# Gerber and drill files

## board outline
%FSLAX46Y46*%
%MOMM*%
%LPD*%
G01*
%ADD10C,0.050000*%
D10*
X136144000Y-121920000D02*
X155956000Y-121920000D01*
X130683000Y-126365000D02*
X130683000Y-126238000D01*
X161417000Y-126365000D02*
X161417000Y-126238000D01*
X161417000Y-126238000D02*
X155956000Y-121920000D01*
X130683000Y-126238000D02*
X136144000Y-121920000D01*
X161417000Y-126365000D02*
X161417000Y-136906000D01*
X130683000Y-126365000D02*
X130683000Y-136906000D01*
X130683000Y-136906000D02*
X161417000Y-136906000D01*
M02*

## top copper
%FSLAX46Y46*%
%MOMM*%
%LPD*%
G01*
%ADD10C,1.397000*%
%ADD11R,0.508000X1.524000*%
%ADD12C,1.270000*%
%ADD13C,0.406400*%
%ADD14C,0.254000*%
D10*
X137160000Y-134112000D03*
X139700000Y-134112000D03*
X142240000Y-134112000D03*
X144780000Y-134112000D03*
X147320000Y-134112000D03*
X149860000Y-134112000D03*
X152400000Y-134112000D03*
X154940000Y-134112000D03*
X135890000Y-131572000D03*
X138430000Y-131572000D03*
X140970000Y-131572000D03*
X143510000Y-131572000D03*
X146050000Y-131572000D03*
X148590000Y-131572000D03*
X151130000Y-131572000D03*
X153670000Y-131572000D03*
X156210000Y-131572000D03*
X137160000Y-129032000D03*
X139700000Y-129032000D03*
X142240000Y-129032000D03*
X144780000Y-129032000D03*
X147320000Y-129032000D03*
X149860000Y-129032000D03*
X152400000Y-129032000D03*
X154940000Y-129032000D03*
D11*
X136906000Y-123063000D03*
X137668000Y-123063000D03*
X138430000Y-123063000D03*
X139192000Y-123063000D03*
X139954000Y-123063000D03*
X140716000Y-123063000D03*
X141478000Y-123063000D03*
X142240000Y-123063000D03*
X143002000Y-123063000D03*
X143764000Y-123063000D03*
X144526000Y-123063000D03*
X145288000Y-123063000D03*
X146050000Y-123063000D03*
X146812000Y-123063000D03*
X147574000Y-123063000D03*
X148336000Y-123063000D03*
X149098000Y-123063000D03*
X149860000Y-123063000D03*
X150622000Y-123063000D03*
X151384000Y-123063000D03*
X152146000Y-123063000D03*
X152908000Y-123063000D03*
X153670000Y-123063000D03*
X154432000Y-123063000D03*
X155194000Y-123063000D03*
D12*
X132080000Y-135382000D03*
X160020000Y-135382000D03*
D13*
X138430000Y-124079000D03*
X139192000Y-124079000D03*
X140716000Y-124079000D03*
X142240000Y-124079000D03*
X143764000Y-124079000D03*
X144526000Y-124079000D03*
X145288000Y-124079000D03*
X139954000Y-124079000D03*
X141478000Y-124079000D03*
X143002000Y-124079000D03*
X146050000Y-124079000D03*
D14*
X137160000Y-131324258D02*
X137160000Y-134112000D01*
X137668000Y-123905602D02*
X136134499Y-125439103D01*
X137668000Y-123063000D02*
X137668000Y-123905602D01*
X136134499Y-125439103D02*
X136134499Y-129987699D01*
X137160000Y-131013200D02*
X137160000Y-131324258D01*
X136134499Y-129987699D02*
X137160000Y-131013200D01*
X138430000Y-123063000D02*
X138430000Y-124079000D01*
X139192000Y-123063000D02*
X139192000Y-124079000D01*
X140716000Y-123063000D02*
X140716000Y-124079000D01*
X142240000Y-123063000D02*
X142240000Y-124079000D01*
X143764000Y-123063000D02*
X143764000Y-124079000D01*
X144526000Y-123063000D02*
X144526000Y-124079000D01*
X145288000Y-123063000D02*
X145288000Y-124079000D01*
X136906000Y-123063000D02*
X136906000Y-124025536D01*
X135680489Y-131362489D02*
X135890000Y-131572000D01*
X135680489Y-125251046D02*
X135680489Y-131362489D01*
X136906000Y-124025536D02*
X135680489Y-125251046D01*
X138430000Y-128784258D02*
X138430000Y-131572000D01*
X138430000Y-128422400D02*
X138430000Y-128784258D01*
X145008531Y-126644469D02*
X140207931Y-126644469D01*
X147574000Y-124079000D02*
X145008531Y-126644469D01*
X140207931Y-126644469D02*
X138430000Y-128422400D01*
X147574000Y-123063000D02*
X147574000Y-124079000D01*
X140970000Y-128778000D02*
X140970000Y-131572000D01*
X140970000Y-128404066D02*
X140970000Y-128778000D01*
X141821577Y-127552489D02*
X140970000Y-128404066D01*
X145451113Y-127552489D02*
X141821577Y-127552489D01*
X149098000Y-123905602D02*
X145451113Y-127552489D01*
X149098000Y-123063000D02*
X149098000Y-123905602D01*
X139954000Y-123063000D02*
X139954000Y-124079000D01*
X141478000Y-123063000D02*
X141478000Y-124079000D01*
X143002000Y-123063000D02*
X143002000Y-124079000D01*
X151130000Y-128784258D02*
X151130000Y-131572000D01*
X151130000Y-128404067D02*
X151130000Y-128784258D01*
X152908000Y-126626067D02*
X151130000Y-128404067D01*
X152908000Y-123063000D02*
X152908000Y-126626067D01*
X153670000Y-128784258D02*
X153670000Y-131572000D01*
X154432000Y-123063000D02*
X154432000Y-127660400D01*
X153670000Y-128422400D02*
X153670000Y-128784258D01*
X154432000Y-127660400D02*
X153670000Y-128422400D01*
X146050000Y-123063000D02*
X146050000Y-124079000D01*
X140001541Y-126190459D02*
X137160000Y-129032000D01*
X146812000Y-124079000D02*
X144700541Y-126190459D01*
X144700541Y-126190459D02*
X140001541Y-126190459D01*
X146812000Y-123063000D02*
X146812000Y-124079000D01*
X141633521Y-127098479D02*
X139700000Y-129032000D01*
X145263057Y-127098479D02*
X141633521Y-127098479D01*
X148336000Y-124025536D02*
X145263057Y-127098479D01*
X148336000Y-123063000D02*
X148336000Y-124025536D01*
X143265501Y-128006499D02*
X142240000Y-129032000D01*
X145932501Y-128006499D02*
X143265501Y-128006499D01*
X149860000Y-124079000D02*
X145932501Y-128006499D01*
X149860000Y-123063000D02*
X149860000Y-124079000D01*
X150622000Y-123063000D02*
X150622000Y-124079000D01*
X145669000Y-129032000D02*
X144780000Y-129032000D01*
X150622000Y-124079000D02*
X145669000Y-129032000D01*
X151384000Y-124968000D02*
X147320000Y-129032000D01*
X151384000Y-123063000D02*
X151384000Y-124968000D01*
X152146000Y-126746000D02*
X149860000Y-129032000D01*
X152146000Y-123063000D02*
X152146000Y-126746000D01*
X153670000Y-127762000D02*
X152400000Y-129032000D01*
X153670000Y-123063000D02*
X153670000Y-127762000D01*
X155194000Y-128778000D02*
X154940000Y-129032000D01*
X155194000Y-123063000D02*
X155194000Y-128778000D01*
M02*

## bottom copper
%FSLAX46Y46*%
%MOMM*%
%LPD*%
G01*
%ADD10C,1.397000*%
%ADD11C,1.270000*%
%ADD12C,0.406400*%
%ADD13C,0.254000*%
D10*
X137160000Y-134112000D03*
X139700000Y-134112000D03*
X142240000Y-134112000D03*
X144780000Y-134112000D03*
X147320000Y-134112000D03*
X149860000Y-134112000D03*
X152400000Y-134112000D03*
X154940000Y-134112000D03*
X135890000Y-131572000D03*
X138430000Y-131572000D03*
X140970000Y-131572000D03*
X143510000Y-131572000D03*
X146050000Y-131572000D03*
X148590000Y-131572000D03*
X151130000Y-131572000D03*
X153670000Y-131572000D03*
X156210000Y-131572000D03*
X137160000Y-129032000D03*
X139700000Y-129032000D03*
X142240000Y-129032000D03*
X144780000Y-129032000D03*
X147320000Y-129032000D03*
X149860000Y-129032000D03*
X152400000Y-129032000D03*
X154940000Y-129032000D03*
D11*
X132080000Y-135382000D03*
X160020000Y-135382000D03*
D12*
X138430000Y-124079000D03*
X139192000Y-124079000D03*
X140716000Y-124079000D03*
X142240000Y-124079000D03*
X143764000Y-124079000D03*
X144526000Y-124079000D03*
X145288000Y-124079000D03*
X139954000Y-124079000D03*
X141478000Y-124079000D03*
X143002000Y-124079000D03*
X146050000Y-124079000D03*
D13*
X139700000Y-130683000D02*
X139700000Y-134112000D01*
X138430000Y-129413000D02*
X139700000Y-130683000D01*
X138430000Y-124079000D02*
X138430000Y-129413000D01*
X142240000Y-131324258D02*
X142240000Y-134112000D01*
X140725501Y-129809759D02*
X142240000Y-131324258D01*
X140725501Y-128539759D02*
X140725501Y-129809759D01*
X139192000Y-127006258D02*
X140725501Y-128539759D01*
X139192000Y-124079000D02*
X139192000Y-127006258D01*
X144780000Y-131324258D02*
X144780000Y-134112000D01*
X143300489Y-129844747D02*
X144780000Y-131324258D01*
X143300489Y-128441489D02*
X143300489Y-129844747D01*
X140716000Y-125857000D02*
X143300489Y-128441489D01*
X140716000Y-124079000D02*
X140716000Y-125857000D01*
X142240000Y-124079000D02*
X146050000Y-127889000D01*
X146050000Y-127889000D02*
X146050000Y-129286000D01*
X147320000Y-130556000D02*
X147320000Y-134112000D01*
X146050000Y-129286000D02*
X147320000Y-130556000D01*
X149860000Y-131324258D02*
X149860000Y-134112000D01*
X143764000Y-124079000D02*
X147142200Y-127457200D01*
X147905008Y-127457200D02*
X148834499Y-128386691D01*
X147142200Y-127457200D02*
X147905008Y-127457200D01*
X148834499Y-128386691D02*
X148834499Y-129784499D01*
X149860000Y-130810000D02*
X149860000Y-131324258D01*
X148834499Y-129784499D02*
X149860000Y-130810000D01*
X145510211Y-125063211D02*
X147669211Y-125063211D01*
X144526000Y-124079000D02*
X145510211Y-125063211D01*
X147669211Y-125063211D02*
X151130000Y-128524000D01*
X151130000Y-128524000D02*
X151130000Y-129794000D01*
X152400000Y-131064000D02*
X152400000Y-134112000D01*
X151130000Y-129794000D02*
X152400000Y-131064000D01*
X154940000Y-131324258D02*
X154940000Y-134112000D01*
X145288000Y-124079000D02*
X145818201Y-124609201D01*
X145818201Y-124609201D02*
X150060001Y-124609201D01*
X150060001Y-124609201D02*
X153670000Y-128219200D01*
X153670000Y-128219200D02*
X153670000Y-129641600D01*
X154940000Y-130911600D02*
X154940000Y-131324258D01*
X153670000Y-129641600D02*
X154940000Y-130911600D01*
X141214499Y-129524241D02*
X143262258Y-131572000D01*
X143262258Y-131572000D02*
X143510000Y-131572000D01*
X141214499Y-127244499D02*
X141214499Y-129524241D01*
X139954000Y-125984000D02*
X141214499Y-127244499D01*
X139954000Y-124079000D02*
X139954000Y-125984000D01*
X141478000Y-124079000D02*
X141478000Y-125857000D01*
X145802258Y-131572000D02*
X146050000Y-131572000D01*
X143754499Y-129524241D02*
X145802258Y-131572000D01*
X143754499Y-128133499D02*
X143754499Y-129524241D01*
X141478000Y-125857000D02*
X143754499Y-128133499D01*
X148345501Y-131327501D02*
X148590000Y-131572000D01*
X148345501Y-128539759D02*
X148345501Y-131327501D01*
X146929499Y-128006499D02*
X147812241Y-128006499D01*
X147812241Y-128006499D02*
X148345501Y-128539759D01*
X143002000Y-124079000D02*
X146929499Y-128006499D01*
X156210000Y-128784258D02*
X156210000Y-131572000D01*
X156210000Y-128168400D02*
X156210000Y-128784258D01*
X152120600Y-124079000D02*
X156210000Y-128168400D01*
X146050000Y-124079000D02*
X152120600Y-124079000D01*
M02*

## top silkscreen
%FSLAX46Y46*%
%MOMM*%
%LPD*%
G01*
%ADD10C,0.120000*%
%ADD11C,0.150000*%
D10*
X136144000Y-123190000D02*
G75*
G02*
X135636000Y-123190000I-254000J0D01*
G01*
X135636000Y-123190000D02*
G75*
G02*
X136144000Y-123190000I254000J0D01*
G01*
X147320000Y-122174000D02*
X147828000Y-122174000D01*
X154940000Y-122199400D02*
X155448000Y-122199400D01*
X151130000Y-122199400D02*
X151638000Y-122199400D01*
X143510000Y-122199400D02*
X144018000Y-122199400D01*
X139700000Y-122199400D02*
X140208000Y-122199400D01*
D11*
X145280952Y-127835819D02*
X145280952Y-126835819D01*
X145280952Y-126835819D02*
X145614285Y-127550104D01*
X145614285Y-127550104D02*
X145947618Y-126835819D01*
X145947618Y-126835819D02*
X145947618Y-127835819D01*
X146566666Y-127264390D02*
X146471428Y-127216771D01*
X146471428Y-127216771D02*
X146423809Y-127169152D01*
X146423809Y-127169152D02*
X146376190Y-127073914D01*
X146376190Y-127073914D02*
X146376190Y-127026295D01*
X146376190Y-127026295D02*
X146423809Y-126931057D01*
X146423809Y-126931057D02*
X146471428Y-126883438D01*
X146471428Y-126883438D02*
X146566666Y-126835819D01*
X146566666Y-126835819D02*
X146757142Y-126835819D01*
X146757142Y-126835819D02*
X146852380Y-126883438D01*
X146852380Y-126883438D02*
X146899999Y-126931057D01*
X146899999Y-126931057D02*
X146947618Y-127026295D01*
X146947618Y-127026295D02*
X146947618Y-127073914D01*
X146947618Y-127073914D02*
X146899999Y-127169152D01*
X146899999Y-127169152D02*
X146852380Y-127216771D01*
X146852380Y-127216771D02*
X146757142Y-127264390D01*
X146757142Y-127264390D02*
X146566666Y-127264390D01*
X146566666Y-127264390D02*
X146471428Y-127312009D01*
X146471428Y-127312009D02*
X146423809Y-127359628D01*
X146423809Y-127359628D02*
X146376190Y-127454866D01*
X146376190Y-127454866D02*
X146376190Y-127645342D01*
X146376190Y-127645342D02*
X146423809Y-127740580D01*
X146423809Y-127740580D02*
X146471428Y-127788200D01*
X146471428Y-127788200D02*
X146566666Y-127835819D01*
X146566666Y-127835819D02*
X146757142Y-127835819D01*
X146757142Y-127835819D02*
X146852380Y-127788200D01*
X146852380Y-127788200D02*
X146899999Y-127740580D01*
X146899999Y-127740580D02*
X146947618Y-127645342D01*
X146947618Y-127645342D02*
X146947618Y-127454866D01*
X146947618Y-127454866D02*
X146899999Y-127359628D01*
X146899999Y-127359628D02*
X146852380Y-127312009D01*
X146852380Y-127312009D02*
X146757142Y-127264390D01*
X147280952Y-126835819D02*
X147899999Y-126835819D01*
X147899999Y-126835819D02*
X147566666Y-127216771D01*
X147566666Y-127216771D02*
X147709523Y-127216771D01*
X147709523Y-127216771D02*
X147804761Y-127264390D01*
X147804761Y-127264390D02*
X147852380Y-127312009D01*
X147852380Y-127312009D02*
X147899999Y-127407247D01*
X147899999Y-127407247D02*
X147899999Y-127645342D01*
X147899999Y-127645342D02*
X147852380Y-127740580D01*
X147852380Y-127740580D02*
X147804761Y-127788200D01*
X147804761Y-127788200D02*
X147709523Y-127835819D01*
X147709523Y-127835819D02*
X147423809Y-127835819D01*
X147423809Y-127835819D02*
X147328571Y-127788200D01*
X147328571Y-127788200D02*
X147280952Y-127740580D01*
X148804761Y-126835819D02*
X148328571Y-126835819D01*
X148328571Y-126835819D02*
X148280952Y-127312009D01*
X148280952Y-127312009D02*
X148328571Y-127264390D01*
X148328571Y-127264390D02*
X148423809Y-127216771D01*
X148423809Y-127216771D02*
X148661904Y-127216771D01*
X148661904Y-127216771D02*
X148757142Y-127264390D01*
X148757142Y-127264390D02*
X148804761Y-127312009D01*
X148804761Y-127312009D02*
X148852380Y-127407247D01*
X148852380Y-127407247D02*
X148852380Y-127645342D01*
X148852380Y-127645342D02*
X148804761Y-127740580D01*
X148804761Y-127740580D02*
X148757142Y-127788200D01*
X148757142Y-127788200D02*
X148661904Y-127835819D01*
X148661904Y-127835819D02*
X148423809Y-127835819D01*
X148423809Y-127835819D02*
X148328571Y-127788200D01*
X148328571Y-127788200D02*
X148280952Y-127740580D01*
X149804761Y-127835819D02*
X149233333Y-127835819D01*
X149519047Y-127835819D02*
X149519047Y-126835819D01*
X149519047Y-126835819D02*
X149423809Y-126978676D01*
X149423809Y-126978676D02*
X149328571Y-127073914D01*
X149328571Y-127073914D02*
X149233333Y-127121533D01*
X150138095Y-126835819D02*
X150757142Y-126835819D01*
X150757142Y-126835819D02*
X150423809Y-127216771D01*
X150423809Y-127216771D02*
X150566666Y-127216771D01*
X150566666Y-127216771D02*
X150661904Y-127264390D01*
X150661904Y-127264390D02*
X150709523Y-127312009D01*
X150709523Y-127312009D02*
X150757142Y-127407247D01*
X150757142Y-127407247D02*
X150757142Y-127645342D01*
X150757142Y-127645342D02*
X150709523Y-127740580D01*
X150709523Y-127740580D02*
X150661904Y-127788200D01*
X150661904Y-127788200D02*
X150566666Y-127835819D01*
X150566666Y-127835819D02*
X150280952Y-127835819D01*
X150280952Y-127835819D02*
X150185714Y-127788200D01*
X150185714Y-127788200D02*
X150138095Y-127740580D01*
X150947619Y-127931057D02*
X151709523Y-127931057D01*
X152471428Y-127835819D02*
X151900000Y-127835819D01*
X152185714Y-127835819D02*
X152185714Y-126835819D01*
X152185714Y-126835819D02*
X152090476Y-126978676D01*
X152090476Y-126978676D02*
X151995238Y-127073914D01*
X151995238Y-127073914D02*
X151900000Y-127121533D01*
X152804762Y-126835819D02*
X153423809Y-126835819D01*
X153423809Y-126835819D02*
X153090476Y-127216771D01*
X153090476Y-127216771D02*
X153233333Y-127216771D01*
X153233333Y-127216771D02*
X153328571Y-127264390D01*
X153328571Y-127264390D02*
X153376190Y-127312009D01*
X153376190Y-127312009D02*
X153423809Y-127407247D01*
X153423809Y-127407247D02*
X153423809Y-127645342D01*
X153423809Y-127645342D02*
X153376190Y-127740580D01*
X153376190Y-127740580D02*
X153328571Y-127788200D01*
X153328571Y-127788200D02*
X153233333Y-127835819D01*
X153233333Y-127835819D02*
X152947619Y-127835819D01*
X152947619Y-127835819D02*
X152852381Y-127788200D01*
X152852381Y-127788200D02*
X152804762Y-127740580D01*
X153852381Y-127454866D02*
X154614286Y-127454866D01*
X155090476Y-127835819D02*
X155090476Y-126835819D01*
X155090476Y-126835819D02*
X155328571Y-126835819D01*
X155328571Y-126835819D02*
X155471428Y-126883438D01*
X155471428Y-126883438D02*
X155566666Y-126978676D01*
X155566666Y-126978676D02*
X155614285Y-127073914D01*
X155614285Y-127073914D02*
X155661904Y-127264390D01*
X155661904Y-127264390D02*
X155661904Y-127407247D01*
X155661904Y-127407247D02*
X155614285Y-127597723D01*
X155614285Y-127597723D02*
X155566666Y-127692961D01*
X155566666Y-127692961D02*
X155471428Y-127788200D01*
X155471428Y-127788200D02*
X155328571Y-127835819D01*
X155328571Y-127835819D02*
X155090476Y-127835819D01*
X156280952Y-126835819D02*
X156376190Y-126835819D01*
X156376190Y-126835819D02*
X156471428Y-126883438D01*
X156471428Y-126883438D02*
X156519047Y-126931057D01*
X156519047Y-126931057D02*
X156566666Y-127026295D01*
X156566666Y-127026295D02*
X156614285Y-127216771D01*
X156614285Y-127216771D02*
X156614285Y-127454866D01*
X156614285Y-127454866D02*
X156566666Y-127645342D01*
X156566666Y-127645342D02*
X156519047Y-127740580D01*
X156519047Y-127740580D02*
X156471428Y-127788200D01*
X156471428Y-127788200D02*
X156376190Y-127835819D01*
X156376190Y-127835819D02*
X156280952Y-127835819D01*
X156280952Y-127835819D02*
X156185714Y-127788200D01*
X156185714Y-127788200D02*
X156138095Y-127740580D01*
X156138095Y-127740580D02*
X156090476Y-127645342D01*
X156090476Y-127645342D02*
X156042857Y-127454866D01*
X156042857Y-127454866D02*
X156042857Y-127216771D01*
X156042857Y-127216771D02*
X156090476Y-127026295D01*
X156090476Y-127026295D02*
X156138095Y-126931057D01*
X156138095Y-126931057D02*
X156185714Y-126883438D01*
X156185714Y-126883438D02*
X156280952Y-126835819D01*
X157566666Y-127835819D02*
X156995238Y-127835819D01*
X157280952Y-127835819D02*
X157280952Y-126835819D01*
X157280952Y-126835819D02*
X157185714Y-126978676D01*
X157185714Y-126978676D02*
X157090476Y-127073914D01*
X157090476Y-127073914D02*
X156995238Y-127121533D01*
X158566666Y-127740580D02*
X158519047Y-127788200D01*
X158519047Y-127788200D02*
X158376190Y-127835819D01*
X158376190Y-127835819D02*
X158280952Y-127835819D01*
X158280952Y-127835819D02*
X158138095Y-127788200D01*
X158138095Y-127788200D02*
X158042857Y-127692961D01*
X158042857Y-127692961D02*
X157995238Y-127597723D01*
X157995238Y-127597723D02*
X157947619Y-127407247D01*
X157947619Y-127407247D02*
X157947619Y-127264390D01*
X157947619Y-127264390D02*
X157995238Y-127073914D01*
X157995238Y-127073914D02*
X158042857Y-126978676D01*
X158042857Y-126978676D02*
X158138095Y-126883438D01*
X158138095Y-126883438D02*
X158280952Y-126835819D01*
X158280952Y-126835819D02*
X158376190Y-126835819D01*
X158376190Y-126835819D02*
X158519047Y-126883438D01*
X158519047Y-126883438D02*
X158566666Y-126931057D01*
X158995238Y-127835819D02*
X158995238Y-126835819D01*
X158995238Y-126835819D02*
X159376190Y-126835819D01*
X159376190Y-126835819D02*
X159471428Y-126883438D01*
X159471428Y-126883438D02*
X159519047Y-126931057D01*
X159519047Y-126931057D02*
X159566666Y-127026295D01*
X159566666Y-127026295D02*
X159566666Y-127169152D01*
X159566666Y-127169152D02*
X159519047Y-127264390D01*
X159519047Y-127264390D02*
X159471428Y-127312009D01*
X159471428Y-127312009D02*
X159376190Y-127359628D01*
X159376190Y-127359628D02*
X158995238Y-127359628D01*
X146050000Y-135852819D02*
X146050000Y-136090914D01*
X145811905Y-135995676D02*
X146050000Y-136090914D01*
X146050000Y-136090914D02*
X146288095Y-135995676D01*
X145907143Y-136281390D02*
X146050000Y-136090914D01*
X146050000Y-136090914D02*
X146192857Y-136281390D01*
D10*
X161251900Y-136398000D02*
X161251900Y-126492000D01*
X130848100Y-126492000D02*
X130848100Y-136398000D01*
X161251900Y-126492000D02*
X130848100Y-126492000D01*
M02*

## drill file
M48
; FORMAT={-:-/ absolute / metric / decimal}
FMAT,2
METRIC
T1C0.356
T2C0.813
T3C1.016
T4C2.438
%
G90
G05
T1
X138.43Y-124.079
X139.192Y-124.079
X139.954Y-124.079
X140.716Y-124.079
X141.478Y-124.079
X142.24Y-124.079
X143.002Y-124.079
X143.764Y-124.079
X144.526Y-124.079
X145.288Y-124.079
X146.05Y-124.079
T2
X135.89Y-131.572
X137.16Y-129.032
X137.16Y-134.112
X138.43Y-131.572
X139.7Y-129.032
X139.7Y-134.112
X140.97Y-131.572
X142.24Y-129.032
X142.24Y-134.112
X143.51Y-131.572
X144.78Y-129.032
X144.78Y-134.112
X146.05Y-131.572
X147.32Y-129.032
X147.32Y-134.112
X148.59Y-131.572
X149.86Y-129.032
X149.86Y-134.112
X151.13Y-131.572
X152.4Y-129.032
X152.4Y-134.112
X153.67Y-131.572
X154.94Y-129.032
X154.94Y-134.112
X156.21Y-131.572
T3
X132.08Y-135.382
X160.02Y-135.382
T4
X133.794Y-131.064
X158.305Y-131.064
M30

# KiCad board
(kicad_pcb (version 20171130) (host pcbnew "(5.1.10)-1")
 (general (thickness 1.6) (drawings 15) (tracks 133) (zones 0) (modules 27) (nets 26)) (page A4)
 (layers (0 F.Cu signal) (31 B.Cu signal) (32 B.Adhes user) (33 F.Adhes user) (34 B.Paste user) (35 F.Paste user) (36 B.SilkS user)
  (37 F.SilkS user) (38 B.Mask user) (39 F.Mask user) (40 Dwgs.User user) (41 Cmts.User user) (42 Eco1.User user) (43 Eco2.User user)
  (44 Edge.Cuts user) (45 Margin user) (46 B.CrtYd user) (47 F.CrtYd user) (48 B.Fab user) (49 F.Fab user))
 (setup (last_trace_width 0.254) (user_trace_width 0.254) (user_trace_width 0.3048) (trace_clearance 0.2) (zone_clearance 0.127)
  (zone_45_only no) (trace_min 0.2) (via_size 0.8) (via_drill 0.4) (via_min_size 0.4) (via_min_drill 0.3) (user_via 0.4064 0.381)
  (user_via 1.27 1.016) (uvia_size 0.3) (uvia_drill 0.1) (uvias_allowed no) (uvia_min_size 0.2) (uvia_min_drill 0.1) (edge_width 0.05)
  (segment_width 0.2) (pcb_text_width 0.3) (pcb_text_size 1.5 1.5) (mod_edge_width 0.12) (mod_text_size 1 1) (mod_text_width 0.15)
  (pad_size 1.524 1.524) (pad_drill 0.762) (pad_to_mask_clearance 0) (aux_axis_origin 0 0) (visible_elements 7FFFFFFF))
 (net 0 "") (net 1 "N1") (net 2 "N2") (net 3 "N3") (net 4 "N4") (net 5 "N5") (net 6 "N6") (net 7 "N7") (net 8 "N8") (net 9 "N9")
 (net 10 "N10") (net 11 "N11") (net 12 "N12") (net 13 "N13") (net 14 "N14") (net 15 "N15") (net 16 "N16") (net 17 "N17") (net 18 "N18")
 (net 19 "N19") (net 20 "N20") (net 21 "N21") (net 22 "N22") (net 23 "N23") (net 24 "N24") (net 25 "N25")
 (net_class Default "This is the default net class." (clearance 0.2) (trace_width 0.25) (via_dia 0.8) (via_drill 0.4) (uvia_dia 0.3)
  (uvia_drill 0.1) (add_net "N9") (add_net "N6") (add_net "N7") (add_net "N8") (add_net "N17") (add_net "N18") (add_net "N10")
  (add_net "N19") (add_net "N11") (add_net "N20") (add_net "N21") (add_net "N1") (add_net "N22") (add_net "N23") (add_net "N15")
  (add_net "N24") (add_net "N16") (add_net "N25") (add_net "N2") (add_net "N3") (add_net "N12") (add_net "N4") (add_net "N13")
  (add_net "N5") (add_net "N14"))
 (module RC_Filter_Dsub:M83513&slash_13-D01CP (layer F.Cu) (at 146.05 137.414 180)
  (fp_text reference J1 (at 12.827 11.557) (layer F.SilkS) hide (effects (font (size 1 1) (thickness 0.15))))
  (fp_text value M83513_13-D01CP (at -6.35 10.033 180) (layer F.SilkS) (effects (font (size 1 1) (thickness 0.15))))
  (fp_line (start -15.2019 1.016) (end -15.2019 10.922) (layer F.SilkS) (width 0.12))
  (fp_line (start 15.2019 10.922) (end 15.2019 1.016) (layer F.SilkS) (width 0.12))
  (fp_line (start -15.2019 10.922) (end 15.2019 10.922) (layer F.SilkS) (width 0.12))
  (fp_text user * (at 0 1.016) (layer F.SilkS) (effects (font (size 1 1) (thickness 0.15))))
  (pad 2 thru_hole circle (at 8.89 3.302 180) (size 1.397 1.397) (drill 0.8128) (layers *.Cu *.Mask) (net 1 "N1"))
  (pad 3 thru_hole circle (at 6.35 3.302 180) (size 1.397 1.397) (drill 0.8128) (layers *.Cu *.Mask) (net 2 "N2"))
  (pad 4 thru_hole circle (at 3.81 3.302 180) (size 1.397 1.397) (drill 0.8128) (layers *.Cu *.Mask) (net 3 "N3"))
  (pad 6 thru_hole circle (at 1.27 3.302 180) (size 1.397 1.397) (drill 0.8128) (layers *.Cu *.Mask) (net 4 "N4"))
  (pad 8 thru_hole circle (at -1.27 3.302 180) (size 1.397 1.397) (drill 0.8128) (layers *.Cu *.Mask) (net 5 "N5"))
  (pad 10 thru_hole circle (at -3.81 3.302 180) (size 1.397 1.397) (drill 0.8128) (layers *.Cu *.Mask) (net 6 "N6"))
  (pad 11 thru_hole circle (at -6.35 3.302 180) (size 1.397 1.397) (drill 0.8128) (layers *.Cu *.Mask) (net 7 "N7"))
  (pad 12 thru_hole circle (at -8.89 3.302 180) (size 1.397 1.397) (drill 0.8128) (layers *.Cu *.Mask) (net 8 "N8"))
  (pad 1 thru_hole circle (at 10.16 5.842 180) (size 1.397 1.397) (drill 0.8128) (layers *.Cu *.Mask) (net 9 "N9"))
  (pad 15 thru_hole circle (at 7.62 5.842 180) (size 1.397 1.397) (drill 0.8128) (layers *.Cu *.Mask) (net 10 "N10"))
  (pad 17 thru_hole circle (at 5.08 5.842 180) (size 1.397 1.397) (drill 0.8128) (layers *.Cu *.Mask) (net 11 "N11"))
  (pad 5 thru_hole circle (at 2.54 5.842 180) (size 1.397 1.397) (drill 0.8128) (layers *.Cu *.Mask) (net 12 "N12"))
  (pad 7 thru_hole circle (at 0 5.842 180) (size 1.397 1.397) (drill 0.8128) (layers *.Cu *.Mask) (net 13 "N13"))
  (pad 9 thru_hole circle (at -2.54 5.842 180) (size 1.397 1.397) (drill 0.8128) (layers *.Cu *.Mask) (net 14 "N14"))
  (pad 22 thru_hole circle (at -5.08 5.842 180) (size 1.397 1.397) (drill 0.8128) (layers *.Cu *.Mask) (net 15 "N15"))
  (pad 24 thru_hole circle (at -7.62 5.842 180) (size 1.397 1.397) (drill 0.8128) (layers *.Cu *.Mask) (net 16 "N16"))
  (pad 13 thru_hole circle (at -10.16 5.842 180) (size 1.397 1.397) (drill 0.8128) (layers *.Cu *.Mask) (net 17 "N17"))
  (pad 14 thru_hole circle (at 8.89 8.382 180) (size 1.397 1.397) (drill 0.8128) (layers *.Cu *.Mask) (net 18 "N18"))
  (pad 16 thru_hole circle (at 6.35 8.382 180) (size 1.397 1.397) (drill 0.8128) (layers *.Cu *.Mask) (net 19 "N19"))
  (pad 18 thru_hole circle (at 3.81 8.382 180) (size 1.397 1.397) (drill 0.8128) (layers *.Cu *.Mask) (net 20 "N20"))
  (pad 19 thru_hole circle (at 1.27 8.382 180) (size 1.397 1.397) (drill 0.8128) (layers *.Cu *.Mask) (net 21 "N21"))
  (pad 20 thru_hole circle (at -1.27 8.382 180) (size 1.397 1.397) (drill 0.8128) (layers *.Cu *.Mask) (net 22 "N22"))
  (pad 21 thru_hole circle (at -3.81 8.382 180) (size 1.397 1.397) (drill 0.8128) (layers *.Cu *.Mask) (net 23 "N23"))
  (pad 23 thru_hole circle (at -6.35 8.382 180) (size 1.397 1.397) (drill 0.8128) (layers *.Cu *.Mask) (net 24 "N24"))
  (pad 25 thru_hole circle (at -8.89 8.382 180) (size 1.397 1.397) (drill 0.8128) (layers *.Cu *.Mask) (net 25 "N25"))
  (pad "" np_thru_hole circle (at -12.2555 6.35 270) (size 2.4384 2.4384) (drill 2.4384) (layers *.Cu *.Mask))
  (pad "" np_thru_hole circle (at 12.2555 6.35 180) (size 2.4384 2.4384) (drill 2.4384) (layers *.Cu *.Mask)))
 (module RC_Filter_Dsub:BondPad (layer F.Cu) (at 136.906 123.063)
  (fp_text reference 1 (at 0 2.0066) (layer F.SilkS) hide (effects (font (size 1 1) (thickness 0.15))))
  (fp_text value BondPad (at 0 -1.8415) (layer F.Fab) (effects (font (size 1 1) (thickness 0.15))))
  (pad 1 smd rect (at 0 0) (size 0.508 1.524) (layers F.Cu F.Paste F.Mask) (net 9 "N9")))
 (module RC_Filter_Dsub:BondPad (layer F.Cu) (at 137.668 123.063)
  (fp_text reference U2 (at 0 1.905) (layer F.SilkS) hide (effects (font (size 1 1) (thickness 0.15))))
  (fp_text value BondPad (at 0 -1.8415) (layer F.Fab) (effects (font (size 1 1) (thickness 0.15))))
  (pad 1 smd rect (at 0 0) (size 0.508 1.524) (layers F.Cu F.Paste F.Mask) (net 1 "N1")))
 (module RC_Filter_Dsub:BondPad (layer F.Cu) (at 138.43 123.063)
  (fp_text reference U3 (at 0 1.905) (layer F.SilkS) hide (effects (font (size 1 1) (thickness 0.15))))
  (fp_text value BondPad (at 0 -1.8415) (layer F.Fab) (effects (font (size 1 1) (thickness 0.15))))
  (pad 1 smd rect (at 0 0) (size 0.508 1.524) (layers F.Cu F.Paste F.Mask) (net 2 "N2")))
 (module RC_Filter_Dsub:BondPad (layer F.Cu) (at 139.192 123.063)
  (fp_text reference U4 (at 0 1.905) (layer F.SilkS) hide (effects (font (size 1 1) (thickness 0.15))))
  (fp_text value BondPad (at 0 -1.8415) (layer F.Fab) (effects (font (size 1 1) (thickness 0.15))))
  (pad 1 smd rect (at 0 0) (size 0.508 1.524) (layers F.Cu F.Paste F.Mask) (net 3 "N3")))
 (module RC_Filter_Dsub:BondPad (layer F.Cu) (at 139.954 123.063)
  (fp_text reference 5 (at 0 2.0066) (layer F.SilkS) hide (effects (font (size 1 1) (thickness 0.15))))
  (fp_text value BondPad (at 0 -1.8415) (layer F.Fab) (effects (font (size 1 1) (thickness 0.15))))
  (pad 1 smd rect (at 0 0) (size 0.508 1.524) (layers F.Cu F.Paste F.Mask) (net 12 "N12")))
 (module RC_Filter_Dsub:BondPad (layer F.Cu) (at 140.716 123.063)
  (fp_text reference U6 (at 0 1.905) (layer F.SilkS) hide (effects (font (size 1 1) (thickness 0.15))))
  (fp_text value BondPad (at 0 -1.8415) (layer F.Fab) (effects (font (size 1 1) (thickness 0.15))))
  (pad 1 smd rect (at 0 0) (size 0.508 1.524) (layers F.Cu F.Paste F.Mask) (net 4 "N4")))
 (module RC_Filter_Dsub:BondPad (layer F.Cu) (at 141.478 123.063)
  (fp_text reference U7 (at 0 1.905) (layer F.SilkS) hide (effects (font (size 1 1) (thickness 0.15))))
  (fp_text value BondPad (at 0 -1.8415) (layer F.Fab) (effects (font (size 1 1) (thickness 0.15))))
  (pad 1 smd rect (at 0 0) (size 0.508 1.524) (layers F.Cu F.Paste F.Mask) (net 13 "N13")))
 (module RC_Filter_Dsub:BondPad (layer F.Cu) (at 142.24 123.063)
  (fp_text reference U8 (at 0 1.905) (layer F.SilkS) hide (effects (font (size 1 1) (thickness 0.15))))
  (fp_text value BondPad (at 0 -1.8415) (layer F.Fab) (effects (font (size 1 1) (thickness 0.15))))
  (pad 1 smd rect (at 0 0) (size 0.508 1.524) (layers F.Cu F.Paste F.Mask) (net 5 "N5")))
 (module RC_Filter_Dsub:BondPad (layer F.Cu) (at 143.002 123.063)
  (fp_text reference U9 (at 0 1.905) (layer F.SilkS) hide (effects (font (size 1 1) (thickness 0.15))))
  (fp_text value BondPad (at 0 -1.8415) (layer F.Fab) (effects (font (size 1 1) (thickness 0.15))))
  (pad 1 smd rect (at 0 0) (size 0.508 1.524) (layers F.Cu F.Paste F.Mask) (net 14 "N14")))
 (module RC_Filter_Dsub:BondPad (layer F.Cu) (at 143.764 123.063)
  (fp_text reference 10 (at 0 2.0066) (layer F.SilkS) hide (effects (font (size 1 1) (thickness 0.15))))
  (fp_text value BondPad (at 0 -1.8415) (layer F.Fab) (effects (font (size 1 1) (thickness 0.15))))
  (pad 1 smd rect (at 0 0) (size 0.508 1.524) (layers F.Cu F.Paste F.Mask) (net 6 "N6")))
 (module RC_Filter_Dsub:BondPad (layer F.Cu) (at 144.526 123.063)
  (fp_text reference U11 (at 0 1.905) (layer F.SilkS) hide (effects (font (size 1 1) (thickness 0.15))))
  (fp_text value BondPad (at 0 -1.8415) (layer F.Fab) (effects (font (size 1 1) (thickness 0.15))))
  (pad 1 smd rect (at 0 0) (size 0.508 1.524) (layers F.Cu F.Paste F.Mask) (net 7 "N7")))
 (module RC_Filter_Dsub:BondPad (layer F.Cu) (at 145.288 123.063)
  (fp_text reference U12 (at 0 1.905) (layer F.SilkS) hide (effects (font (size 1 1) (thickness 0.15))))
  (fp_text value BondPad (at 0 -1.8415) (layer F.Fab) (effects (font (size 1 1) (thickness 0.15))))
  (pad 1 smd rect (at 0 0) (size 0.508 1.524) (layers F.Cu F.Paste F.Mask) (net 8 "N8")))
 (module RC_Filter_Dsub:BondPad (layer F.Cu) (at 146.05 123.063)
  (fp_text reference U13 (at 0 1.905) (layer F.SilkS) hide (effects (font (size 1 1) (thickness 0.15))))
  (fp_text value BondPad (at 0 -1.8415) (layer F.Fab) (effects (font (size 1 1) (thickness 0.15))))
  (pad 1 smd rect (at 0 0) (size 0.508 1.524) (layers F.Cu F.Paste F.Mask) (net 17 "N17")))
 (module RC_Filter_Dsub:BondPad (layer F.Cu) (at 146.812 123.063)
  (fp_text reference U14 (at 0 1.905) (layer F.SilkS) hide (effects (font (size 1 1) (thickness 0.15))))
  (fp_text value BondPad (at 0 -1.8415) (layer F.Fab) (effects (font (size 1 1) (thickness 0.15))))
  (pad 1 smd rect (at 0 0) (size 0.508 1.524) (layers F.Cu F.Paste F.Mask) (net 18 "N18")))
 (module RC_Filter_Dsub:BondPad (layer F.Cu) (at 147.574 123.063)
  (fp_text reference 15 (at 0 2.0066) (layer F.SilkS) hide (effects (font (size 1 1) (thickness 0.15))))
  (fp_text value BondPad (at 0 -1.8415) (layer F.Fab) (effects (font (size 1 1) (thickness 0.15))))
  (pad 1 smd rect (at 0 0) (size 0.508 1.524) (layers F.Cu F.Paste F.Mask) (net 10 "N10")))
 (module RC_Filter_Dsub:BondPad (layer F.Cu) (at 148.336 123.063)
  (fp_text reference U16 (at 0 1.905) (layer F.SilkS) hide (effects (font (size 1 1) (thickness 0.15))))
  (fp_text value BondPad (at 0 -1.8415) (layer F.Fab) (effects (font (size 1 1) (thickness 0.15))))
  (pad 1 smd rect (at 0 0) (size 0.508 1.524) (layers F.Cu F.Paste F.Mask) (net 19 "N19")))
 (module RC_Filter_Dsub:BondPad (layer F.Cu) (at 149.098 123.063)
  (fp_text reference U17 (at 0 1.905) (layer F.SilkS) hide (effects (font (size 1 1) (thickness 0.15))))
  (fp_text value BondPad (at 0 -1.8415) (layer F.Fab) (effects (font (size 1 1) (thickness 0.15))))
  (pad 1 smd rect (at 0 0) (size 0.508 1.524) (layers F.Cu F.Paste F.Mask) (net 11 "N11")))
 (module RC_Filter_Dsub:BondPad (layer F.Cu) (at 149.86 123.063)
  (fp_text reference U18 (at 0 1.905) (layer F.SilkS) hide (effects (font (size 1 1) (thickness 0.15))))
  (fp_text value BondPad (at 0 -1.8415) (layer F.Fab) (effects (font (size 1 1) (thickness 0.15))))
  (pad 1 smd rect (at 0 0) (size 0.508 1.524) (layers F.Cu F.Paste F.Mask) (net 20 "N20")))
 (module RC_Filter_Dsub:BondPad (layer F.Cu) (at 150.622 123.063)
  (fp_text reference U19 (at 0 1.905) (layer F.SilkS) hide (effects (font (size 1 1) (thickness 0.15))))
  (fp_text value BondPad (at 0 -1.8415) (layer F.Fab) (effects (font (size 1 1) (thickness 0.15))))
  (pad 1 smd rect (at 0 0) (size 0.508 1.524) (layers F.Cu F.Paste F.Mask) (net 21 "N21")))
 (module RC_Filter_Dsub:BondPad (layer F.Cu) (at 151.384 123.063)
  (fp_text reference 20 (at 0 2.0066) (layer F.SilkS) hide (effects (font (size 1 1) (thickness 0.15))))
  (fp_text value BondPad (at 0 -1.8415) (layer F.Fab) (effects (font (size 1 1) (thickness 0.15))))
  (pad 1 smd rect (at 0 0) (size 0.508 1.524) (layers F.Cu F.Paste F.Mask) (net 22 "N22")))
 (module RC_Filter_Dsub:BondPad (layer F.Cu) (at 152.146 123.063)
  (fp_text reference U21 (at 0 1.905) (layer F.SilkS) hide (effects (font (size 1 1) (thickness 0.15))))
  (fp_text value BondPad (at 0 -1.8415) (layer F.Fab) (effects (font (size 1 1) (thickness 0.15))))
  (pad 1 smd rect (at 0 0) (size 0.508 1.524) (layers F.Cu F.Paste F.Mask) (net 23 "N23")))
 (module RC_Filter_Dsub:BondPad (layer F.Cu) (at 152.908 123.063)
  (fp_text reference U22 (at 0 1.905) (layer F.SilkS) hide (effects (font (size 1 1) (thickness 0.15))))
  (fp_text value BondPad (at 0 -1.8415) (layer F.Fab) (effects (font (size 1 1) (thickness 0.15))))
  (pad 1 smd rect (at 0 0) (size 0.508 1.524) (layers F.Cu F.Paste F.Mask) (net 15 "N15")))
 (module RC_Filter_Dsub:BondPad (layer F.Cu) (at 153.67 123.063)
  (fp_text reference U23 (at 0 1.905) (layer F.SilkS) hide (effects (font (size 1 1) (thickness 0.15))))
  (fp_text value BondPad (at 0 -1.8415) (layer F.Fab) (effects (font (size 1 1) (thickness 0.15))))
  (pad 1 smd rect (at 0 0) (size 0.508 1.524) (layers F.Cu F.Paste F.Mask) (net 24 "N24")))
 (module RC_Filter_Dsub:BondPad (layer F.Cu) (at 154.432 123.063)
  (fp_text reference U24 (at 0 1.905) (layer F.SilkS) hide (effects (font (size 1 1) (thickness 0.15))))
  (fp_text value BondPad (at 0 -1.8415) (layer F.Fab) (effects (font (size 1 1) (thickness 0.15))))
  (pad 1 smd rect (at 0 0) (size 0.508 1.524) (layers F.Cu F.Paste F.Mask) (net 16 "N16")))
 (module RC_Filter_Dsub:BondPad (layer F.Cu) (at 155.194 123.063)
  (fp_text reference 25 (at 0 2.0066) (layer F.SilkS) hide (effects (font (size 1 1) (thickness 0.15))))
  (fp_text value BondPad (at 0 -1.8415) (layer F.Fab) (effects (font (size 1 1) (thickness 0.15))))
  (pad 1 smd rect (at 0 0) (size 0.508 1.524) (layers F.Cu F.Paste F.Mask) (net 25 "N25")))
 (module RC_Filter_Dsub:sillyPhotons (layer F.Cu) (at 133.35 127.254)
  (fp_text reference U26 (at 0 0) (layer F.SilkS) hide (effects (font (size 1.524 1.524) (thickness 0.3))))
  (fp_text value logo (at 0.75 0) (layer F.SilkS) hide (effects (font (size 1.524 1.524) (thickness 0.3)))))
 (gr_circle (center 135.89 123.19) (end 135.89 122.936) (layer F.SilkS) (width 0.12))
 (gr_line (start 147.32 122.174) (end 147.828 122.174) (layer F.SilkS) (width 0.12))
 (gr_line (start 154.94 122.1994) (end 155.448 122.1994) (layer F.SilkS) (width 0.12))
 (gr_line (start 151.13 122.1994) (end 151.638 122.1994) (layer F.SilkS) (width 0.12))
 (gr_line (start 143.51 122.1994) (end 144.018 122.1994) (layer F.SilkS) (width 0.12))
 (gr_line (start 139.7 122.1994) (end 140.208 122.1994) (layer F.SilkS) (width 0.12))
 (gr_line (start 136.144 121.92) (end 155.956 121.92) (layer Edge.Cuts) (width 0.05))
 (gr_line (start 130.683 126.365) (end 130.683 126.238) (layer Edge.Cuts) (width 0.05))
 (gr_line (start 161.417 126.365) (end 161.417 126.238) (layer Edge.Cuts) (width 0.05))
 (gr_line (start 161.417 126.238) (end 155.956 121.92) (layer Edge.Cuts) (width 0.05))
 (gr_line (start 130.683 126.238) (end 136.144 121.92) (layer Edge.Cuts) (width 0.05))
 (gr_line (start 161.417 126.365) (end 161.417 136.906) (layer Edge.Cuts) (width 0.05))
 (gr_line (start 130.683 126.365) (end 130.683 136.906) (layer Edge.Cuts) (width 0.05))
 (gr_line (start 130.683 136.906) (end 161.417 136.906) (layer Edge.Cuts) (width 0.05))
 (via (at 132.08 135.382) (size 1.27) (drill 1.016) (layers F.Cu B.Cu) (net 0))
 (via (at 160.02 135.382) (size 1.27) (drill 1.016) (layers F.Cu B.Cu) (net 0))
 (segment (start 137.16 131.324258) (end 137.16 134.112) (width 0.254) (layer F.Cu) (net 1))
 (segment (start 137.668 123.905602) (end 136.134499 125.439103) (width 0.254) (layer F.Cu) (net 1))
 (segment (start 137.668 123.063) (end 137.668 123.905602) (width 0.254) (layer F.Cu) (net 1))
 (segment (start 136.134499 125.439103) (end 136.134499 129.987699) (width 0.254) (layer F.Cu) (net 1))
 (segment (start 137.16 131.0132) (end 137.16 131.324258) (width 0.254) (layer F.Cu) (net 1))
 (segment (start 136.134499 129.987699) (end 137.16 131.0132) (width 0.254) (layer F.Cu) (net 1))
 (via (at 138.43 124.079) (size 0.4064) (drill 0.3556) (layers F.Cu B.Cu) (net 2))
 (segment (start 138.43 123.063) (end 138.43 124.079) (width 0.254) (layer F.Cu) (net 2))
 (segment (start 139.7 130.683) (end 139.7 134.112) (width 0.254) (layer B.Cu) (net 2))
 (segment (start 138.43 129.413) (end 139.7 130.683) (width 0.254) (layer B.Cu) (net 2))
 (segment (start 138.43 124.079) (end 138.43 129.413) (width 0.254) (layer B.Cu) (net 2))
 (via (at 139.192 124.079) (size 0.4064) (drill 0.3556) (layers F.Cu B.Cu) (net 3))
 (segment (start 139.192 123.063) (end 139.192 124.079) (width 0.254) (layer F.Cu) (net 3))
 (segment (start 142.24 131.324258) (end 142.24 134.112) (width 0.254) (layer B.Cu) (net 3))
 (segment (start 140.725501 129.809759) (end 142.24 131.324258) (width 0.254) (layer B.Cu) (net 3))
 (segment (start 140.725501 128.539759) (end 140.725501 129.809759) (width 0.254) (layer B.Cu) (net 3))
 (segment (start 139.192 127.006258) (end 140.725501 128.539759) (width 0.254) (layer B.Cu) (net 3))
 (segment (start 139.192 124.079) (end 139.192 127.006258) (width 0.254) (layer B.Cu) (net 3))
 (via (at 140.716 124.079) (size 0.4064) (drill 0.3556) (layers F.Cu B.Cu) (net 4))
 (segment (start 140.716 123.063) (end 140.716 124.079) (width 0.254) (layer F.Cu) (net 4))
 (segment (start 144.78 131.324258) (end 144.78 134.112) (width 0.254) (layer B.Cu) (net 4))
 (segment (start 143.300489 129.844747) (end 144.78 131.324258) (width 0.254) (layer B.Cu) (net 4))
 (segment (start 143.300489 128.441489) (end 143.300489 129.844747) (width 0.254) (layer B.Cu) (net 4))
 (segment (start 140.716 125.857) (end 143.300489 128.441489) (width 0.254) (layer B.Cu) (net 4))
 (segment (start 140.716 124.079) (end 140.716 125.857) (width 0.254) (layer B.Cu) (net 4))
 (via (at 142.24 124.079) (size 0.4064) (drill 0.3556) (layers F.Cu B.Cu) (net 5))
 (segment (start 142.24 123.063) (end 142.24 124.079) (width 0.254) (layer F.Cu) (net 5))
 (segment (start 142.24 124.079) (end 146.05 127.889) (width 0.254) (layer B.Cu) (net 5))
 (segment (start 146.05 127.889) (end 146.05 129.286) (width 0.254) (layer B.Cu) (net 5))
 (segment (start 147.32 130.556) (end 147.32 134.112) (width 0.254) (layer B.Cu) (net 5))
 (segment (start 146.05 129.286) (end 147.32 130.556) (width 0.254) (layer B.Cu) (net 5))
 (via (at 143.764 124.079) (size 0.4064) (drill 0.3556) (layers F.Cu B.Cu) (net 6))
 (segment (start 143.764 123.063) (end 143.764 124.079) (width 0.254) (layer F.Cu) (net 6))
 (segment (start 149.86 131.324258) (end 149.86 134.112) (width 0.254) (layer B.Cu) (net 6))
 (segment (start 143.764 124.079) (end 147.1422 127.4572) (width 0.254) (layer B.Cu) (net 6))
 (segment (start 147.905008 127.4572) (end 148.834499 128.386691) (width 0.254) (layer B.Cu) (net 6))
 (segment (start 147.1422 127.4572) (end 147.905008 127.4572) (width 0.254) (layer B.Cu) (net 6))
 (segment (start 148.834499 128.386691) (end 148.834499 129.784499) (width 0.254) (layer B.Cu) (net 6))
 (segment (start 149.86 130.81) (end 149.86 131.324258) (width 0.254) (layer B.Cu) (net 6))
 (segment (start 148.834499 129.784499) (end 149.86 130.81) (width 0.254) (layer B.Cu) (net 6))
 (via (at 144.526 124.079) (size 0.4064) (drill 0.3556) (layers F.Cu B.Cu) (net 7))
 (segment (start 144.526 123.063) (end 144.526 124.079) (width 0.254) (layer F.Cu) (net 7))
 (segment (start 145.510211 125.063211) (end 147.669211 125.063211) (width 0.254) (layer B.Cu) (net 7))
 (segment (start 144.526 124.079) (end 145.510211 125.063211) (width 0.254) (layer B.Cu) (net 7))
 (segment (start 147.669211 125.063211) (end 151.13 128.524) (width 0.254) (layer B.Cu) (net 7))
 (segment (start 151.13 128.524) (end 151.13 129.794) (width 0.254) (layer B.Cu) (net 7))
 (segment (start 152.4 131.064) (end 152.4 134.112) (width 0.254) (layer B.Cu) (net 7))
 (segment (start 151.13 129.794) (end 152.4 131.064) (width 0.254) (layer B.Cu) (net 7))
 (segment (start 145.288 123.063) (end 145.288 124.079) (width 0.254) (layer F.Cu) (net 8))
 (via (at 145.288 124.079) (size 0.4064) (drill 0.3556) (layers F.Cu B.Cu) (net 8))
 (segment (start 154.94 131.324258) (end 154.94 134.112) (width 0.254) (layer B.Cu) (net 8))
 (segment (start 145.288 124.079) (end 145.818201 124.609201) (width 0.254) (layer B.Cu) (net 8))
 (segment (start 145.818201 124.609201) (end 150.060001 124.609201) (width 0.254) (layer B.Cu) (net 8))
 (segment (start 150.060001 124.609201) (end 153.67 128.2192) (width 0.254) (layer B.Cu) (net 8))
 (segment (start 153.67 128.2192) (end 153.67 129.6416) (width 0.254) (layer B.Cu) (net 8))
 (segment (start 154.94 130.9116) (end 154.94 131.324258) (width 0.254) (layer B.Cu) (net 8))
 (segment (start 153.67 129.6416) (end 154.94 130.9116) (width 0.254) (layer B.Cu) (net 8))
 (segment (start 136.906 123.063) (end 136.906 124.025536) (width 0.254) (layer F.Cu) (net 9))
 (segment (start 135.680489 131.362489) (end 135.89 131.572) (width 0.254) (layer F.Cu) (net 9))
 (segment (start 135.680489 125.251046) (end 135.680489 131.362489) (width 0.254) (layer F.Cu) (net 9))
 (segment (start 136.906 124.025536) (end 135.680489 125.251046) (width 0.254) (layer F.Cu) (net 9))
 (segment (start 138.43 128.784258) (end 138.43 131.572) (width 0.254) (layer F.Cu) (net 10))
 (segment (start 138.43 128.4224) (end 138.43 128.784258) (width 0.254) (layer F.Cu) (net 10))
 (segment (start 145.008531 126.644469) (end 140.207931 126.644469) (width 0.254) (layer F.Cu) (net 10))
 (segment (start 147.574 124.079) (end 145.008531 126.644469) (width 0.254) (layer F.Cu) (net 10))
 (segment (start 140.207931 126.644469) (end 138.43 128.4224) (width 0.254) (layer F.Cu) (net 10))
 (segment (start 147.574 123.063) (end 147.574 124.079) (width 0.254) (layer F.Cu) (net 10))
 (segment (start 140.97 128.778) (end 140.97 131.572) (width 0.254) (layer F.Cu) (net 11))
 (segment (start 140.97 128.404066) (end 140.97 128.778) (width 0.254) (layer F.Cu) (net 11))
 (segment (start 141.821577 127.552489) (end 140.97 128.404066) (width 0.254) (layer F.Cu) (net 11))
 (segment (start 145.451113 127.552489) (end 141.821577 127.552489) (width 0.254) (layer F.Cu) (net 11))
 (segment (start 149.098 123.905602) (end 145.451113 127.552489) (width 0.254) (layer F.Cu) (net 11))
 (segment (start 149.098 123.063) (end 149.098 123.905602) (width 0.254) (layer F.Cu) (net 11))
 (via (at 139.954 124.079) (size 0.4064) (drill 0.3556) (layers F.Cu B.Cu) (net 12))
 (segment (start 139.954 123.063) (end 139.954 124.079) (width 0.254) (layer F.Cu) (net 12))
 (segment (start 141.214499 129.524241) (end 143.262258 131.572) (width 0.254) (layer B.Cu) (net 12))
 (segment (start 143.262258 131.572) (end 143.51 131.572) (width 0.254) (layer B.Cu) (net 12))
 (segment (start 141.214499 127.244499) (end 141.214499 129.524241) (width 0.254) (layer B.Cu) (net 12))
 (segment (start 139.954 125.984) (end 141.214499 127.244499) (width 0.254) (layer B.Cu) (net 12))
 (segment (start 139.954 124.079) (end 139.954 125.984) (width 0.254) (layer B.Cu) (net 12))
 (via (at 141.478 124.079) (size 0.4064) (drill 0.3556) (layers F.Cu B.Cu) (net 13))
 (segment (start 141.478 123.063) (end 141.478 124.079) (width 0.254) (layer F.Cu) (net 13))
 (segment (start 141.478 124.079) (end 141.478 125.857) (width 0.254) (layer B.Cu) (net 13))
 (segment (start 145.802258 131.572) (end 146.05 131.572) (width 0.254) (layer B.Cu) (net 13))
 (segment (start 143.754499 129.524241) (end 145.802258 131.572) (width 0.254) (layer B.Cu) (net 13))
 (segment (start 143.754499 128.133499) (end 143.754499 129.524241) (width 0.254) (layer B.Cu) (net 13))
 (segment (start 141.478 125.857) (end 143.754499 128.133499) (width 0.254) (layer B.Cu) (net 13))
 (via (at 143.002 124.079) (size 0.4064) (drill 0.3556) (layers F.Cu B.Cu) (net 14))
 (segment (start 143.002 123.063) (end 143.002 124.079) (width 0.254) (layer F.Cu) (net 14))
 (segment (start 148.345501 131.327501) (end 148.59 131.572) (width 0.254) (layer B.Cu) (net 14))
 (segment (start 148.345501 128.539759) (end 148.345501 131.327501) (width 0.254) (layer B.Cu) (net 14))
 (segment (start 146.929499 128.006499) (end 147.812241 128.006499) (width 0.254) (layer B.Cu) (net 14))
 (segment (start 147.812241 128.006499) (end 148.345501 128.539759) (width 0.254) (layer B.Cu) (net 14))
 (segment (start 143.002 124.079) (end 146.929499 128.006499) (width 0.254) (layer B.Cu) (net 14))
 (segment (start 151.13 128.784258) (end 151.13 131.572) (width 0.254) (layer F.Cu) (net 15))
 (segment (start 151.13 128.404067) (end 151.13 128.784258) (width 0.254) (layer F.Cu) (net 15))
 (segment (start 152.908 126.626067) (end 151.13 128.404067) (width 0.254) (layer F.Cu) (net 15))
 (segment (start 152.908 123.063) (end 152.908 126.626067) (width 0.254) (layer F.Cu) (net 15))
 (segment (start 153.67 128.784258) (end 153.67 131.572) (width 0.254) (layer F.Cu) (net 16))
 (segment (start 154.432 123.063) (end 154.432 127.6604) (width 0.254) (layer F.Cu) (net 16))
 (segment (start 153.67 128.4224) (end 153.67 128.784258) (width 0.254) (layer F.Cu) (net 16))
 (segment (start 154.432 127.6604) (end 153.67 128.4224) (width 0.254) (layer F.Cu) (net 16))
 (via (at 146.05 124.079) (size 0.4064) (drill 0.3556) (layers F.Cu B.Cu) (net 17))
 (segment (start 146.05 123.063) (end 146.05 124.079) (width 0.254) (layer F.Cu) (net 17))
 (segment (start 156.21 128.784258) (end 156.21 131.572) (width 0.254) (layer B.Cu) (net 17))
 (segment (start 156.21 128.1684) (end 156.21 128.784258) (width 0.254) (layer B.Cu) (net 17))
 (segment (start 152.1206 124.079) (end 156.21 128.1684) (width 0.254) (layer B.Cu) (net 17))
 (segment (start 146.05 124.079) (end 152.1206 124.079) (width 0.254) (layer B.Cu) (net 17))
 (segment (start 140.001541 126.190459) (end 137.16 129.032) (width 0.254) (layer F.Cu) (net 18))
 (segment (start 146.812 124.079) (end 144.700541 126.190459) (width 0.254) (layer F.Cu) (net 18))
 (segment (start 144.700541 126.190459) (end 140.001541 126.190459) (width 0.254) (layer F.Cu) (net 18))
 (segment (start 146.812 123.063) (end 146.812 124.079) (width 0.254) (layer F.Cu) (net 18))
 (segment (start 141.633521 127.098479) (end 139.7 129.032) (width 0.254) (layer F.Cu) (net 19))
 (segment (start 145.263057 127.098479) (end 141.633521 127.098479) (width 0.254) (layer F.Cu) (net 19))
 (segment (start 148.336 124.025536) (end 145.263057 127.098479) (width 0.254) (layer F.Cu) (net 19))
 (segment (start 148.336 123.063) (end 148.336 124.025536) (width 0.254) (layer F.Cu) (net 19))
 (segment (start 143.265501 128.006499) (end 142.24 129.032) (width 0.254) (layer F.Cu) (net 20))
 (segment (start 145.932501 128.006499) (end 143.265501 128.006499) (width 0.254) (layer F.Cu) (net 20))
 (segment (start 149.86 124.079) (end 145.932501 128.006499) (width 0.254) (layer F.Cu) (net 20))
 (segment (start 149.86 123.063) (end 149.86 124.079) (width 0.254) (layer F.Cu) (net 20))
 (segment (start 150.622 123.063) (end 150.622 124.079) (width 0.254) (layer F.Cu) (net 21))
 (segment (start 145.669 129.032) (end 144.78 129.032) (width 0.254) (layer F.Cu) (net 21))
 (segment (start 150.622 124.079) (end 145.669 129.032) (width 0.254) (layer F.Cu) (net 21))
 (segment (start 151.384 124.968) (end 147.32 129.032) (width 0.254) (layer F.Cu) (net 22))
 (segment (start 151.384 123.063) (end 151.384 124.968) (width 0.254) (layer F.Cu) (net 22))
 (segment (start 152.146 126.746) (end 149.86 129.032) (width 0.254) (layer F.Cu) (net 23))
 (segment (start 152.146 123.063) (end 152.146 126.746) (width 0.254) (layer F.Cu) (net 23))
 (segment (start 153.67 127.762) (end 152.4 129.032) (width 0.254) (layer F.Cu) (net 24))
 (segment (start 153.67 123.063) (end 153.67 127.762) (width 0.254) (layer F.Cu) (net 24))
 (segment (start 155.194 128.778) (end 154.94 129.032) (width 0.254) (layer F.Cu) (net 25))
 (segment (start 155.194 123.063) (end 155.194 128.778) (width 0.254) (layer F.Cu) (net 25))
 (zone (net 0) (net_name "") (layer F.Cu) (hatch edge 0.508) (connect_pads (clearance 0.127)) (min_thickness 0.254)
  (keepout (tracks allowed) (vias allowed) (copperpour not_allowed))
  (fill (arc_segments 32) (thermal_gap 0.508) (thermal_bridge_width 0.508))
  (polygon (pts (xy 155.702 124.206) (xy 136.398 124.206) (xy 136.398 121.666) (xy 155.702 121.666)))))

